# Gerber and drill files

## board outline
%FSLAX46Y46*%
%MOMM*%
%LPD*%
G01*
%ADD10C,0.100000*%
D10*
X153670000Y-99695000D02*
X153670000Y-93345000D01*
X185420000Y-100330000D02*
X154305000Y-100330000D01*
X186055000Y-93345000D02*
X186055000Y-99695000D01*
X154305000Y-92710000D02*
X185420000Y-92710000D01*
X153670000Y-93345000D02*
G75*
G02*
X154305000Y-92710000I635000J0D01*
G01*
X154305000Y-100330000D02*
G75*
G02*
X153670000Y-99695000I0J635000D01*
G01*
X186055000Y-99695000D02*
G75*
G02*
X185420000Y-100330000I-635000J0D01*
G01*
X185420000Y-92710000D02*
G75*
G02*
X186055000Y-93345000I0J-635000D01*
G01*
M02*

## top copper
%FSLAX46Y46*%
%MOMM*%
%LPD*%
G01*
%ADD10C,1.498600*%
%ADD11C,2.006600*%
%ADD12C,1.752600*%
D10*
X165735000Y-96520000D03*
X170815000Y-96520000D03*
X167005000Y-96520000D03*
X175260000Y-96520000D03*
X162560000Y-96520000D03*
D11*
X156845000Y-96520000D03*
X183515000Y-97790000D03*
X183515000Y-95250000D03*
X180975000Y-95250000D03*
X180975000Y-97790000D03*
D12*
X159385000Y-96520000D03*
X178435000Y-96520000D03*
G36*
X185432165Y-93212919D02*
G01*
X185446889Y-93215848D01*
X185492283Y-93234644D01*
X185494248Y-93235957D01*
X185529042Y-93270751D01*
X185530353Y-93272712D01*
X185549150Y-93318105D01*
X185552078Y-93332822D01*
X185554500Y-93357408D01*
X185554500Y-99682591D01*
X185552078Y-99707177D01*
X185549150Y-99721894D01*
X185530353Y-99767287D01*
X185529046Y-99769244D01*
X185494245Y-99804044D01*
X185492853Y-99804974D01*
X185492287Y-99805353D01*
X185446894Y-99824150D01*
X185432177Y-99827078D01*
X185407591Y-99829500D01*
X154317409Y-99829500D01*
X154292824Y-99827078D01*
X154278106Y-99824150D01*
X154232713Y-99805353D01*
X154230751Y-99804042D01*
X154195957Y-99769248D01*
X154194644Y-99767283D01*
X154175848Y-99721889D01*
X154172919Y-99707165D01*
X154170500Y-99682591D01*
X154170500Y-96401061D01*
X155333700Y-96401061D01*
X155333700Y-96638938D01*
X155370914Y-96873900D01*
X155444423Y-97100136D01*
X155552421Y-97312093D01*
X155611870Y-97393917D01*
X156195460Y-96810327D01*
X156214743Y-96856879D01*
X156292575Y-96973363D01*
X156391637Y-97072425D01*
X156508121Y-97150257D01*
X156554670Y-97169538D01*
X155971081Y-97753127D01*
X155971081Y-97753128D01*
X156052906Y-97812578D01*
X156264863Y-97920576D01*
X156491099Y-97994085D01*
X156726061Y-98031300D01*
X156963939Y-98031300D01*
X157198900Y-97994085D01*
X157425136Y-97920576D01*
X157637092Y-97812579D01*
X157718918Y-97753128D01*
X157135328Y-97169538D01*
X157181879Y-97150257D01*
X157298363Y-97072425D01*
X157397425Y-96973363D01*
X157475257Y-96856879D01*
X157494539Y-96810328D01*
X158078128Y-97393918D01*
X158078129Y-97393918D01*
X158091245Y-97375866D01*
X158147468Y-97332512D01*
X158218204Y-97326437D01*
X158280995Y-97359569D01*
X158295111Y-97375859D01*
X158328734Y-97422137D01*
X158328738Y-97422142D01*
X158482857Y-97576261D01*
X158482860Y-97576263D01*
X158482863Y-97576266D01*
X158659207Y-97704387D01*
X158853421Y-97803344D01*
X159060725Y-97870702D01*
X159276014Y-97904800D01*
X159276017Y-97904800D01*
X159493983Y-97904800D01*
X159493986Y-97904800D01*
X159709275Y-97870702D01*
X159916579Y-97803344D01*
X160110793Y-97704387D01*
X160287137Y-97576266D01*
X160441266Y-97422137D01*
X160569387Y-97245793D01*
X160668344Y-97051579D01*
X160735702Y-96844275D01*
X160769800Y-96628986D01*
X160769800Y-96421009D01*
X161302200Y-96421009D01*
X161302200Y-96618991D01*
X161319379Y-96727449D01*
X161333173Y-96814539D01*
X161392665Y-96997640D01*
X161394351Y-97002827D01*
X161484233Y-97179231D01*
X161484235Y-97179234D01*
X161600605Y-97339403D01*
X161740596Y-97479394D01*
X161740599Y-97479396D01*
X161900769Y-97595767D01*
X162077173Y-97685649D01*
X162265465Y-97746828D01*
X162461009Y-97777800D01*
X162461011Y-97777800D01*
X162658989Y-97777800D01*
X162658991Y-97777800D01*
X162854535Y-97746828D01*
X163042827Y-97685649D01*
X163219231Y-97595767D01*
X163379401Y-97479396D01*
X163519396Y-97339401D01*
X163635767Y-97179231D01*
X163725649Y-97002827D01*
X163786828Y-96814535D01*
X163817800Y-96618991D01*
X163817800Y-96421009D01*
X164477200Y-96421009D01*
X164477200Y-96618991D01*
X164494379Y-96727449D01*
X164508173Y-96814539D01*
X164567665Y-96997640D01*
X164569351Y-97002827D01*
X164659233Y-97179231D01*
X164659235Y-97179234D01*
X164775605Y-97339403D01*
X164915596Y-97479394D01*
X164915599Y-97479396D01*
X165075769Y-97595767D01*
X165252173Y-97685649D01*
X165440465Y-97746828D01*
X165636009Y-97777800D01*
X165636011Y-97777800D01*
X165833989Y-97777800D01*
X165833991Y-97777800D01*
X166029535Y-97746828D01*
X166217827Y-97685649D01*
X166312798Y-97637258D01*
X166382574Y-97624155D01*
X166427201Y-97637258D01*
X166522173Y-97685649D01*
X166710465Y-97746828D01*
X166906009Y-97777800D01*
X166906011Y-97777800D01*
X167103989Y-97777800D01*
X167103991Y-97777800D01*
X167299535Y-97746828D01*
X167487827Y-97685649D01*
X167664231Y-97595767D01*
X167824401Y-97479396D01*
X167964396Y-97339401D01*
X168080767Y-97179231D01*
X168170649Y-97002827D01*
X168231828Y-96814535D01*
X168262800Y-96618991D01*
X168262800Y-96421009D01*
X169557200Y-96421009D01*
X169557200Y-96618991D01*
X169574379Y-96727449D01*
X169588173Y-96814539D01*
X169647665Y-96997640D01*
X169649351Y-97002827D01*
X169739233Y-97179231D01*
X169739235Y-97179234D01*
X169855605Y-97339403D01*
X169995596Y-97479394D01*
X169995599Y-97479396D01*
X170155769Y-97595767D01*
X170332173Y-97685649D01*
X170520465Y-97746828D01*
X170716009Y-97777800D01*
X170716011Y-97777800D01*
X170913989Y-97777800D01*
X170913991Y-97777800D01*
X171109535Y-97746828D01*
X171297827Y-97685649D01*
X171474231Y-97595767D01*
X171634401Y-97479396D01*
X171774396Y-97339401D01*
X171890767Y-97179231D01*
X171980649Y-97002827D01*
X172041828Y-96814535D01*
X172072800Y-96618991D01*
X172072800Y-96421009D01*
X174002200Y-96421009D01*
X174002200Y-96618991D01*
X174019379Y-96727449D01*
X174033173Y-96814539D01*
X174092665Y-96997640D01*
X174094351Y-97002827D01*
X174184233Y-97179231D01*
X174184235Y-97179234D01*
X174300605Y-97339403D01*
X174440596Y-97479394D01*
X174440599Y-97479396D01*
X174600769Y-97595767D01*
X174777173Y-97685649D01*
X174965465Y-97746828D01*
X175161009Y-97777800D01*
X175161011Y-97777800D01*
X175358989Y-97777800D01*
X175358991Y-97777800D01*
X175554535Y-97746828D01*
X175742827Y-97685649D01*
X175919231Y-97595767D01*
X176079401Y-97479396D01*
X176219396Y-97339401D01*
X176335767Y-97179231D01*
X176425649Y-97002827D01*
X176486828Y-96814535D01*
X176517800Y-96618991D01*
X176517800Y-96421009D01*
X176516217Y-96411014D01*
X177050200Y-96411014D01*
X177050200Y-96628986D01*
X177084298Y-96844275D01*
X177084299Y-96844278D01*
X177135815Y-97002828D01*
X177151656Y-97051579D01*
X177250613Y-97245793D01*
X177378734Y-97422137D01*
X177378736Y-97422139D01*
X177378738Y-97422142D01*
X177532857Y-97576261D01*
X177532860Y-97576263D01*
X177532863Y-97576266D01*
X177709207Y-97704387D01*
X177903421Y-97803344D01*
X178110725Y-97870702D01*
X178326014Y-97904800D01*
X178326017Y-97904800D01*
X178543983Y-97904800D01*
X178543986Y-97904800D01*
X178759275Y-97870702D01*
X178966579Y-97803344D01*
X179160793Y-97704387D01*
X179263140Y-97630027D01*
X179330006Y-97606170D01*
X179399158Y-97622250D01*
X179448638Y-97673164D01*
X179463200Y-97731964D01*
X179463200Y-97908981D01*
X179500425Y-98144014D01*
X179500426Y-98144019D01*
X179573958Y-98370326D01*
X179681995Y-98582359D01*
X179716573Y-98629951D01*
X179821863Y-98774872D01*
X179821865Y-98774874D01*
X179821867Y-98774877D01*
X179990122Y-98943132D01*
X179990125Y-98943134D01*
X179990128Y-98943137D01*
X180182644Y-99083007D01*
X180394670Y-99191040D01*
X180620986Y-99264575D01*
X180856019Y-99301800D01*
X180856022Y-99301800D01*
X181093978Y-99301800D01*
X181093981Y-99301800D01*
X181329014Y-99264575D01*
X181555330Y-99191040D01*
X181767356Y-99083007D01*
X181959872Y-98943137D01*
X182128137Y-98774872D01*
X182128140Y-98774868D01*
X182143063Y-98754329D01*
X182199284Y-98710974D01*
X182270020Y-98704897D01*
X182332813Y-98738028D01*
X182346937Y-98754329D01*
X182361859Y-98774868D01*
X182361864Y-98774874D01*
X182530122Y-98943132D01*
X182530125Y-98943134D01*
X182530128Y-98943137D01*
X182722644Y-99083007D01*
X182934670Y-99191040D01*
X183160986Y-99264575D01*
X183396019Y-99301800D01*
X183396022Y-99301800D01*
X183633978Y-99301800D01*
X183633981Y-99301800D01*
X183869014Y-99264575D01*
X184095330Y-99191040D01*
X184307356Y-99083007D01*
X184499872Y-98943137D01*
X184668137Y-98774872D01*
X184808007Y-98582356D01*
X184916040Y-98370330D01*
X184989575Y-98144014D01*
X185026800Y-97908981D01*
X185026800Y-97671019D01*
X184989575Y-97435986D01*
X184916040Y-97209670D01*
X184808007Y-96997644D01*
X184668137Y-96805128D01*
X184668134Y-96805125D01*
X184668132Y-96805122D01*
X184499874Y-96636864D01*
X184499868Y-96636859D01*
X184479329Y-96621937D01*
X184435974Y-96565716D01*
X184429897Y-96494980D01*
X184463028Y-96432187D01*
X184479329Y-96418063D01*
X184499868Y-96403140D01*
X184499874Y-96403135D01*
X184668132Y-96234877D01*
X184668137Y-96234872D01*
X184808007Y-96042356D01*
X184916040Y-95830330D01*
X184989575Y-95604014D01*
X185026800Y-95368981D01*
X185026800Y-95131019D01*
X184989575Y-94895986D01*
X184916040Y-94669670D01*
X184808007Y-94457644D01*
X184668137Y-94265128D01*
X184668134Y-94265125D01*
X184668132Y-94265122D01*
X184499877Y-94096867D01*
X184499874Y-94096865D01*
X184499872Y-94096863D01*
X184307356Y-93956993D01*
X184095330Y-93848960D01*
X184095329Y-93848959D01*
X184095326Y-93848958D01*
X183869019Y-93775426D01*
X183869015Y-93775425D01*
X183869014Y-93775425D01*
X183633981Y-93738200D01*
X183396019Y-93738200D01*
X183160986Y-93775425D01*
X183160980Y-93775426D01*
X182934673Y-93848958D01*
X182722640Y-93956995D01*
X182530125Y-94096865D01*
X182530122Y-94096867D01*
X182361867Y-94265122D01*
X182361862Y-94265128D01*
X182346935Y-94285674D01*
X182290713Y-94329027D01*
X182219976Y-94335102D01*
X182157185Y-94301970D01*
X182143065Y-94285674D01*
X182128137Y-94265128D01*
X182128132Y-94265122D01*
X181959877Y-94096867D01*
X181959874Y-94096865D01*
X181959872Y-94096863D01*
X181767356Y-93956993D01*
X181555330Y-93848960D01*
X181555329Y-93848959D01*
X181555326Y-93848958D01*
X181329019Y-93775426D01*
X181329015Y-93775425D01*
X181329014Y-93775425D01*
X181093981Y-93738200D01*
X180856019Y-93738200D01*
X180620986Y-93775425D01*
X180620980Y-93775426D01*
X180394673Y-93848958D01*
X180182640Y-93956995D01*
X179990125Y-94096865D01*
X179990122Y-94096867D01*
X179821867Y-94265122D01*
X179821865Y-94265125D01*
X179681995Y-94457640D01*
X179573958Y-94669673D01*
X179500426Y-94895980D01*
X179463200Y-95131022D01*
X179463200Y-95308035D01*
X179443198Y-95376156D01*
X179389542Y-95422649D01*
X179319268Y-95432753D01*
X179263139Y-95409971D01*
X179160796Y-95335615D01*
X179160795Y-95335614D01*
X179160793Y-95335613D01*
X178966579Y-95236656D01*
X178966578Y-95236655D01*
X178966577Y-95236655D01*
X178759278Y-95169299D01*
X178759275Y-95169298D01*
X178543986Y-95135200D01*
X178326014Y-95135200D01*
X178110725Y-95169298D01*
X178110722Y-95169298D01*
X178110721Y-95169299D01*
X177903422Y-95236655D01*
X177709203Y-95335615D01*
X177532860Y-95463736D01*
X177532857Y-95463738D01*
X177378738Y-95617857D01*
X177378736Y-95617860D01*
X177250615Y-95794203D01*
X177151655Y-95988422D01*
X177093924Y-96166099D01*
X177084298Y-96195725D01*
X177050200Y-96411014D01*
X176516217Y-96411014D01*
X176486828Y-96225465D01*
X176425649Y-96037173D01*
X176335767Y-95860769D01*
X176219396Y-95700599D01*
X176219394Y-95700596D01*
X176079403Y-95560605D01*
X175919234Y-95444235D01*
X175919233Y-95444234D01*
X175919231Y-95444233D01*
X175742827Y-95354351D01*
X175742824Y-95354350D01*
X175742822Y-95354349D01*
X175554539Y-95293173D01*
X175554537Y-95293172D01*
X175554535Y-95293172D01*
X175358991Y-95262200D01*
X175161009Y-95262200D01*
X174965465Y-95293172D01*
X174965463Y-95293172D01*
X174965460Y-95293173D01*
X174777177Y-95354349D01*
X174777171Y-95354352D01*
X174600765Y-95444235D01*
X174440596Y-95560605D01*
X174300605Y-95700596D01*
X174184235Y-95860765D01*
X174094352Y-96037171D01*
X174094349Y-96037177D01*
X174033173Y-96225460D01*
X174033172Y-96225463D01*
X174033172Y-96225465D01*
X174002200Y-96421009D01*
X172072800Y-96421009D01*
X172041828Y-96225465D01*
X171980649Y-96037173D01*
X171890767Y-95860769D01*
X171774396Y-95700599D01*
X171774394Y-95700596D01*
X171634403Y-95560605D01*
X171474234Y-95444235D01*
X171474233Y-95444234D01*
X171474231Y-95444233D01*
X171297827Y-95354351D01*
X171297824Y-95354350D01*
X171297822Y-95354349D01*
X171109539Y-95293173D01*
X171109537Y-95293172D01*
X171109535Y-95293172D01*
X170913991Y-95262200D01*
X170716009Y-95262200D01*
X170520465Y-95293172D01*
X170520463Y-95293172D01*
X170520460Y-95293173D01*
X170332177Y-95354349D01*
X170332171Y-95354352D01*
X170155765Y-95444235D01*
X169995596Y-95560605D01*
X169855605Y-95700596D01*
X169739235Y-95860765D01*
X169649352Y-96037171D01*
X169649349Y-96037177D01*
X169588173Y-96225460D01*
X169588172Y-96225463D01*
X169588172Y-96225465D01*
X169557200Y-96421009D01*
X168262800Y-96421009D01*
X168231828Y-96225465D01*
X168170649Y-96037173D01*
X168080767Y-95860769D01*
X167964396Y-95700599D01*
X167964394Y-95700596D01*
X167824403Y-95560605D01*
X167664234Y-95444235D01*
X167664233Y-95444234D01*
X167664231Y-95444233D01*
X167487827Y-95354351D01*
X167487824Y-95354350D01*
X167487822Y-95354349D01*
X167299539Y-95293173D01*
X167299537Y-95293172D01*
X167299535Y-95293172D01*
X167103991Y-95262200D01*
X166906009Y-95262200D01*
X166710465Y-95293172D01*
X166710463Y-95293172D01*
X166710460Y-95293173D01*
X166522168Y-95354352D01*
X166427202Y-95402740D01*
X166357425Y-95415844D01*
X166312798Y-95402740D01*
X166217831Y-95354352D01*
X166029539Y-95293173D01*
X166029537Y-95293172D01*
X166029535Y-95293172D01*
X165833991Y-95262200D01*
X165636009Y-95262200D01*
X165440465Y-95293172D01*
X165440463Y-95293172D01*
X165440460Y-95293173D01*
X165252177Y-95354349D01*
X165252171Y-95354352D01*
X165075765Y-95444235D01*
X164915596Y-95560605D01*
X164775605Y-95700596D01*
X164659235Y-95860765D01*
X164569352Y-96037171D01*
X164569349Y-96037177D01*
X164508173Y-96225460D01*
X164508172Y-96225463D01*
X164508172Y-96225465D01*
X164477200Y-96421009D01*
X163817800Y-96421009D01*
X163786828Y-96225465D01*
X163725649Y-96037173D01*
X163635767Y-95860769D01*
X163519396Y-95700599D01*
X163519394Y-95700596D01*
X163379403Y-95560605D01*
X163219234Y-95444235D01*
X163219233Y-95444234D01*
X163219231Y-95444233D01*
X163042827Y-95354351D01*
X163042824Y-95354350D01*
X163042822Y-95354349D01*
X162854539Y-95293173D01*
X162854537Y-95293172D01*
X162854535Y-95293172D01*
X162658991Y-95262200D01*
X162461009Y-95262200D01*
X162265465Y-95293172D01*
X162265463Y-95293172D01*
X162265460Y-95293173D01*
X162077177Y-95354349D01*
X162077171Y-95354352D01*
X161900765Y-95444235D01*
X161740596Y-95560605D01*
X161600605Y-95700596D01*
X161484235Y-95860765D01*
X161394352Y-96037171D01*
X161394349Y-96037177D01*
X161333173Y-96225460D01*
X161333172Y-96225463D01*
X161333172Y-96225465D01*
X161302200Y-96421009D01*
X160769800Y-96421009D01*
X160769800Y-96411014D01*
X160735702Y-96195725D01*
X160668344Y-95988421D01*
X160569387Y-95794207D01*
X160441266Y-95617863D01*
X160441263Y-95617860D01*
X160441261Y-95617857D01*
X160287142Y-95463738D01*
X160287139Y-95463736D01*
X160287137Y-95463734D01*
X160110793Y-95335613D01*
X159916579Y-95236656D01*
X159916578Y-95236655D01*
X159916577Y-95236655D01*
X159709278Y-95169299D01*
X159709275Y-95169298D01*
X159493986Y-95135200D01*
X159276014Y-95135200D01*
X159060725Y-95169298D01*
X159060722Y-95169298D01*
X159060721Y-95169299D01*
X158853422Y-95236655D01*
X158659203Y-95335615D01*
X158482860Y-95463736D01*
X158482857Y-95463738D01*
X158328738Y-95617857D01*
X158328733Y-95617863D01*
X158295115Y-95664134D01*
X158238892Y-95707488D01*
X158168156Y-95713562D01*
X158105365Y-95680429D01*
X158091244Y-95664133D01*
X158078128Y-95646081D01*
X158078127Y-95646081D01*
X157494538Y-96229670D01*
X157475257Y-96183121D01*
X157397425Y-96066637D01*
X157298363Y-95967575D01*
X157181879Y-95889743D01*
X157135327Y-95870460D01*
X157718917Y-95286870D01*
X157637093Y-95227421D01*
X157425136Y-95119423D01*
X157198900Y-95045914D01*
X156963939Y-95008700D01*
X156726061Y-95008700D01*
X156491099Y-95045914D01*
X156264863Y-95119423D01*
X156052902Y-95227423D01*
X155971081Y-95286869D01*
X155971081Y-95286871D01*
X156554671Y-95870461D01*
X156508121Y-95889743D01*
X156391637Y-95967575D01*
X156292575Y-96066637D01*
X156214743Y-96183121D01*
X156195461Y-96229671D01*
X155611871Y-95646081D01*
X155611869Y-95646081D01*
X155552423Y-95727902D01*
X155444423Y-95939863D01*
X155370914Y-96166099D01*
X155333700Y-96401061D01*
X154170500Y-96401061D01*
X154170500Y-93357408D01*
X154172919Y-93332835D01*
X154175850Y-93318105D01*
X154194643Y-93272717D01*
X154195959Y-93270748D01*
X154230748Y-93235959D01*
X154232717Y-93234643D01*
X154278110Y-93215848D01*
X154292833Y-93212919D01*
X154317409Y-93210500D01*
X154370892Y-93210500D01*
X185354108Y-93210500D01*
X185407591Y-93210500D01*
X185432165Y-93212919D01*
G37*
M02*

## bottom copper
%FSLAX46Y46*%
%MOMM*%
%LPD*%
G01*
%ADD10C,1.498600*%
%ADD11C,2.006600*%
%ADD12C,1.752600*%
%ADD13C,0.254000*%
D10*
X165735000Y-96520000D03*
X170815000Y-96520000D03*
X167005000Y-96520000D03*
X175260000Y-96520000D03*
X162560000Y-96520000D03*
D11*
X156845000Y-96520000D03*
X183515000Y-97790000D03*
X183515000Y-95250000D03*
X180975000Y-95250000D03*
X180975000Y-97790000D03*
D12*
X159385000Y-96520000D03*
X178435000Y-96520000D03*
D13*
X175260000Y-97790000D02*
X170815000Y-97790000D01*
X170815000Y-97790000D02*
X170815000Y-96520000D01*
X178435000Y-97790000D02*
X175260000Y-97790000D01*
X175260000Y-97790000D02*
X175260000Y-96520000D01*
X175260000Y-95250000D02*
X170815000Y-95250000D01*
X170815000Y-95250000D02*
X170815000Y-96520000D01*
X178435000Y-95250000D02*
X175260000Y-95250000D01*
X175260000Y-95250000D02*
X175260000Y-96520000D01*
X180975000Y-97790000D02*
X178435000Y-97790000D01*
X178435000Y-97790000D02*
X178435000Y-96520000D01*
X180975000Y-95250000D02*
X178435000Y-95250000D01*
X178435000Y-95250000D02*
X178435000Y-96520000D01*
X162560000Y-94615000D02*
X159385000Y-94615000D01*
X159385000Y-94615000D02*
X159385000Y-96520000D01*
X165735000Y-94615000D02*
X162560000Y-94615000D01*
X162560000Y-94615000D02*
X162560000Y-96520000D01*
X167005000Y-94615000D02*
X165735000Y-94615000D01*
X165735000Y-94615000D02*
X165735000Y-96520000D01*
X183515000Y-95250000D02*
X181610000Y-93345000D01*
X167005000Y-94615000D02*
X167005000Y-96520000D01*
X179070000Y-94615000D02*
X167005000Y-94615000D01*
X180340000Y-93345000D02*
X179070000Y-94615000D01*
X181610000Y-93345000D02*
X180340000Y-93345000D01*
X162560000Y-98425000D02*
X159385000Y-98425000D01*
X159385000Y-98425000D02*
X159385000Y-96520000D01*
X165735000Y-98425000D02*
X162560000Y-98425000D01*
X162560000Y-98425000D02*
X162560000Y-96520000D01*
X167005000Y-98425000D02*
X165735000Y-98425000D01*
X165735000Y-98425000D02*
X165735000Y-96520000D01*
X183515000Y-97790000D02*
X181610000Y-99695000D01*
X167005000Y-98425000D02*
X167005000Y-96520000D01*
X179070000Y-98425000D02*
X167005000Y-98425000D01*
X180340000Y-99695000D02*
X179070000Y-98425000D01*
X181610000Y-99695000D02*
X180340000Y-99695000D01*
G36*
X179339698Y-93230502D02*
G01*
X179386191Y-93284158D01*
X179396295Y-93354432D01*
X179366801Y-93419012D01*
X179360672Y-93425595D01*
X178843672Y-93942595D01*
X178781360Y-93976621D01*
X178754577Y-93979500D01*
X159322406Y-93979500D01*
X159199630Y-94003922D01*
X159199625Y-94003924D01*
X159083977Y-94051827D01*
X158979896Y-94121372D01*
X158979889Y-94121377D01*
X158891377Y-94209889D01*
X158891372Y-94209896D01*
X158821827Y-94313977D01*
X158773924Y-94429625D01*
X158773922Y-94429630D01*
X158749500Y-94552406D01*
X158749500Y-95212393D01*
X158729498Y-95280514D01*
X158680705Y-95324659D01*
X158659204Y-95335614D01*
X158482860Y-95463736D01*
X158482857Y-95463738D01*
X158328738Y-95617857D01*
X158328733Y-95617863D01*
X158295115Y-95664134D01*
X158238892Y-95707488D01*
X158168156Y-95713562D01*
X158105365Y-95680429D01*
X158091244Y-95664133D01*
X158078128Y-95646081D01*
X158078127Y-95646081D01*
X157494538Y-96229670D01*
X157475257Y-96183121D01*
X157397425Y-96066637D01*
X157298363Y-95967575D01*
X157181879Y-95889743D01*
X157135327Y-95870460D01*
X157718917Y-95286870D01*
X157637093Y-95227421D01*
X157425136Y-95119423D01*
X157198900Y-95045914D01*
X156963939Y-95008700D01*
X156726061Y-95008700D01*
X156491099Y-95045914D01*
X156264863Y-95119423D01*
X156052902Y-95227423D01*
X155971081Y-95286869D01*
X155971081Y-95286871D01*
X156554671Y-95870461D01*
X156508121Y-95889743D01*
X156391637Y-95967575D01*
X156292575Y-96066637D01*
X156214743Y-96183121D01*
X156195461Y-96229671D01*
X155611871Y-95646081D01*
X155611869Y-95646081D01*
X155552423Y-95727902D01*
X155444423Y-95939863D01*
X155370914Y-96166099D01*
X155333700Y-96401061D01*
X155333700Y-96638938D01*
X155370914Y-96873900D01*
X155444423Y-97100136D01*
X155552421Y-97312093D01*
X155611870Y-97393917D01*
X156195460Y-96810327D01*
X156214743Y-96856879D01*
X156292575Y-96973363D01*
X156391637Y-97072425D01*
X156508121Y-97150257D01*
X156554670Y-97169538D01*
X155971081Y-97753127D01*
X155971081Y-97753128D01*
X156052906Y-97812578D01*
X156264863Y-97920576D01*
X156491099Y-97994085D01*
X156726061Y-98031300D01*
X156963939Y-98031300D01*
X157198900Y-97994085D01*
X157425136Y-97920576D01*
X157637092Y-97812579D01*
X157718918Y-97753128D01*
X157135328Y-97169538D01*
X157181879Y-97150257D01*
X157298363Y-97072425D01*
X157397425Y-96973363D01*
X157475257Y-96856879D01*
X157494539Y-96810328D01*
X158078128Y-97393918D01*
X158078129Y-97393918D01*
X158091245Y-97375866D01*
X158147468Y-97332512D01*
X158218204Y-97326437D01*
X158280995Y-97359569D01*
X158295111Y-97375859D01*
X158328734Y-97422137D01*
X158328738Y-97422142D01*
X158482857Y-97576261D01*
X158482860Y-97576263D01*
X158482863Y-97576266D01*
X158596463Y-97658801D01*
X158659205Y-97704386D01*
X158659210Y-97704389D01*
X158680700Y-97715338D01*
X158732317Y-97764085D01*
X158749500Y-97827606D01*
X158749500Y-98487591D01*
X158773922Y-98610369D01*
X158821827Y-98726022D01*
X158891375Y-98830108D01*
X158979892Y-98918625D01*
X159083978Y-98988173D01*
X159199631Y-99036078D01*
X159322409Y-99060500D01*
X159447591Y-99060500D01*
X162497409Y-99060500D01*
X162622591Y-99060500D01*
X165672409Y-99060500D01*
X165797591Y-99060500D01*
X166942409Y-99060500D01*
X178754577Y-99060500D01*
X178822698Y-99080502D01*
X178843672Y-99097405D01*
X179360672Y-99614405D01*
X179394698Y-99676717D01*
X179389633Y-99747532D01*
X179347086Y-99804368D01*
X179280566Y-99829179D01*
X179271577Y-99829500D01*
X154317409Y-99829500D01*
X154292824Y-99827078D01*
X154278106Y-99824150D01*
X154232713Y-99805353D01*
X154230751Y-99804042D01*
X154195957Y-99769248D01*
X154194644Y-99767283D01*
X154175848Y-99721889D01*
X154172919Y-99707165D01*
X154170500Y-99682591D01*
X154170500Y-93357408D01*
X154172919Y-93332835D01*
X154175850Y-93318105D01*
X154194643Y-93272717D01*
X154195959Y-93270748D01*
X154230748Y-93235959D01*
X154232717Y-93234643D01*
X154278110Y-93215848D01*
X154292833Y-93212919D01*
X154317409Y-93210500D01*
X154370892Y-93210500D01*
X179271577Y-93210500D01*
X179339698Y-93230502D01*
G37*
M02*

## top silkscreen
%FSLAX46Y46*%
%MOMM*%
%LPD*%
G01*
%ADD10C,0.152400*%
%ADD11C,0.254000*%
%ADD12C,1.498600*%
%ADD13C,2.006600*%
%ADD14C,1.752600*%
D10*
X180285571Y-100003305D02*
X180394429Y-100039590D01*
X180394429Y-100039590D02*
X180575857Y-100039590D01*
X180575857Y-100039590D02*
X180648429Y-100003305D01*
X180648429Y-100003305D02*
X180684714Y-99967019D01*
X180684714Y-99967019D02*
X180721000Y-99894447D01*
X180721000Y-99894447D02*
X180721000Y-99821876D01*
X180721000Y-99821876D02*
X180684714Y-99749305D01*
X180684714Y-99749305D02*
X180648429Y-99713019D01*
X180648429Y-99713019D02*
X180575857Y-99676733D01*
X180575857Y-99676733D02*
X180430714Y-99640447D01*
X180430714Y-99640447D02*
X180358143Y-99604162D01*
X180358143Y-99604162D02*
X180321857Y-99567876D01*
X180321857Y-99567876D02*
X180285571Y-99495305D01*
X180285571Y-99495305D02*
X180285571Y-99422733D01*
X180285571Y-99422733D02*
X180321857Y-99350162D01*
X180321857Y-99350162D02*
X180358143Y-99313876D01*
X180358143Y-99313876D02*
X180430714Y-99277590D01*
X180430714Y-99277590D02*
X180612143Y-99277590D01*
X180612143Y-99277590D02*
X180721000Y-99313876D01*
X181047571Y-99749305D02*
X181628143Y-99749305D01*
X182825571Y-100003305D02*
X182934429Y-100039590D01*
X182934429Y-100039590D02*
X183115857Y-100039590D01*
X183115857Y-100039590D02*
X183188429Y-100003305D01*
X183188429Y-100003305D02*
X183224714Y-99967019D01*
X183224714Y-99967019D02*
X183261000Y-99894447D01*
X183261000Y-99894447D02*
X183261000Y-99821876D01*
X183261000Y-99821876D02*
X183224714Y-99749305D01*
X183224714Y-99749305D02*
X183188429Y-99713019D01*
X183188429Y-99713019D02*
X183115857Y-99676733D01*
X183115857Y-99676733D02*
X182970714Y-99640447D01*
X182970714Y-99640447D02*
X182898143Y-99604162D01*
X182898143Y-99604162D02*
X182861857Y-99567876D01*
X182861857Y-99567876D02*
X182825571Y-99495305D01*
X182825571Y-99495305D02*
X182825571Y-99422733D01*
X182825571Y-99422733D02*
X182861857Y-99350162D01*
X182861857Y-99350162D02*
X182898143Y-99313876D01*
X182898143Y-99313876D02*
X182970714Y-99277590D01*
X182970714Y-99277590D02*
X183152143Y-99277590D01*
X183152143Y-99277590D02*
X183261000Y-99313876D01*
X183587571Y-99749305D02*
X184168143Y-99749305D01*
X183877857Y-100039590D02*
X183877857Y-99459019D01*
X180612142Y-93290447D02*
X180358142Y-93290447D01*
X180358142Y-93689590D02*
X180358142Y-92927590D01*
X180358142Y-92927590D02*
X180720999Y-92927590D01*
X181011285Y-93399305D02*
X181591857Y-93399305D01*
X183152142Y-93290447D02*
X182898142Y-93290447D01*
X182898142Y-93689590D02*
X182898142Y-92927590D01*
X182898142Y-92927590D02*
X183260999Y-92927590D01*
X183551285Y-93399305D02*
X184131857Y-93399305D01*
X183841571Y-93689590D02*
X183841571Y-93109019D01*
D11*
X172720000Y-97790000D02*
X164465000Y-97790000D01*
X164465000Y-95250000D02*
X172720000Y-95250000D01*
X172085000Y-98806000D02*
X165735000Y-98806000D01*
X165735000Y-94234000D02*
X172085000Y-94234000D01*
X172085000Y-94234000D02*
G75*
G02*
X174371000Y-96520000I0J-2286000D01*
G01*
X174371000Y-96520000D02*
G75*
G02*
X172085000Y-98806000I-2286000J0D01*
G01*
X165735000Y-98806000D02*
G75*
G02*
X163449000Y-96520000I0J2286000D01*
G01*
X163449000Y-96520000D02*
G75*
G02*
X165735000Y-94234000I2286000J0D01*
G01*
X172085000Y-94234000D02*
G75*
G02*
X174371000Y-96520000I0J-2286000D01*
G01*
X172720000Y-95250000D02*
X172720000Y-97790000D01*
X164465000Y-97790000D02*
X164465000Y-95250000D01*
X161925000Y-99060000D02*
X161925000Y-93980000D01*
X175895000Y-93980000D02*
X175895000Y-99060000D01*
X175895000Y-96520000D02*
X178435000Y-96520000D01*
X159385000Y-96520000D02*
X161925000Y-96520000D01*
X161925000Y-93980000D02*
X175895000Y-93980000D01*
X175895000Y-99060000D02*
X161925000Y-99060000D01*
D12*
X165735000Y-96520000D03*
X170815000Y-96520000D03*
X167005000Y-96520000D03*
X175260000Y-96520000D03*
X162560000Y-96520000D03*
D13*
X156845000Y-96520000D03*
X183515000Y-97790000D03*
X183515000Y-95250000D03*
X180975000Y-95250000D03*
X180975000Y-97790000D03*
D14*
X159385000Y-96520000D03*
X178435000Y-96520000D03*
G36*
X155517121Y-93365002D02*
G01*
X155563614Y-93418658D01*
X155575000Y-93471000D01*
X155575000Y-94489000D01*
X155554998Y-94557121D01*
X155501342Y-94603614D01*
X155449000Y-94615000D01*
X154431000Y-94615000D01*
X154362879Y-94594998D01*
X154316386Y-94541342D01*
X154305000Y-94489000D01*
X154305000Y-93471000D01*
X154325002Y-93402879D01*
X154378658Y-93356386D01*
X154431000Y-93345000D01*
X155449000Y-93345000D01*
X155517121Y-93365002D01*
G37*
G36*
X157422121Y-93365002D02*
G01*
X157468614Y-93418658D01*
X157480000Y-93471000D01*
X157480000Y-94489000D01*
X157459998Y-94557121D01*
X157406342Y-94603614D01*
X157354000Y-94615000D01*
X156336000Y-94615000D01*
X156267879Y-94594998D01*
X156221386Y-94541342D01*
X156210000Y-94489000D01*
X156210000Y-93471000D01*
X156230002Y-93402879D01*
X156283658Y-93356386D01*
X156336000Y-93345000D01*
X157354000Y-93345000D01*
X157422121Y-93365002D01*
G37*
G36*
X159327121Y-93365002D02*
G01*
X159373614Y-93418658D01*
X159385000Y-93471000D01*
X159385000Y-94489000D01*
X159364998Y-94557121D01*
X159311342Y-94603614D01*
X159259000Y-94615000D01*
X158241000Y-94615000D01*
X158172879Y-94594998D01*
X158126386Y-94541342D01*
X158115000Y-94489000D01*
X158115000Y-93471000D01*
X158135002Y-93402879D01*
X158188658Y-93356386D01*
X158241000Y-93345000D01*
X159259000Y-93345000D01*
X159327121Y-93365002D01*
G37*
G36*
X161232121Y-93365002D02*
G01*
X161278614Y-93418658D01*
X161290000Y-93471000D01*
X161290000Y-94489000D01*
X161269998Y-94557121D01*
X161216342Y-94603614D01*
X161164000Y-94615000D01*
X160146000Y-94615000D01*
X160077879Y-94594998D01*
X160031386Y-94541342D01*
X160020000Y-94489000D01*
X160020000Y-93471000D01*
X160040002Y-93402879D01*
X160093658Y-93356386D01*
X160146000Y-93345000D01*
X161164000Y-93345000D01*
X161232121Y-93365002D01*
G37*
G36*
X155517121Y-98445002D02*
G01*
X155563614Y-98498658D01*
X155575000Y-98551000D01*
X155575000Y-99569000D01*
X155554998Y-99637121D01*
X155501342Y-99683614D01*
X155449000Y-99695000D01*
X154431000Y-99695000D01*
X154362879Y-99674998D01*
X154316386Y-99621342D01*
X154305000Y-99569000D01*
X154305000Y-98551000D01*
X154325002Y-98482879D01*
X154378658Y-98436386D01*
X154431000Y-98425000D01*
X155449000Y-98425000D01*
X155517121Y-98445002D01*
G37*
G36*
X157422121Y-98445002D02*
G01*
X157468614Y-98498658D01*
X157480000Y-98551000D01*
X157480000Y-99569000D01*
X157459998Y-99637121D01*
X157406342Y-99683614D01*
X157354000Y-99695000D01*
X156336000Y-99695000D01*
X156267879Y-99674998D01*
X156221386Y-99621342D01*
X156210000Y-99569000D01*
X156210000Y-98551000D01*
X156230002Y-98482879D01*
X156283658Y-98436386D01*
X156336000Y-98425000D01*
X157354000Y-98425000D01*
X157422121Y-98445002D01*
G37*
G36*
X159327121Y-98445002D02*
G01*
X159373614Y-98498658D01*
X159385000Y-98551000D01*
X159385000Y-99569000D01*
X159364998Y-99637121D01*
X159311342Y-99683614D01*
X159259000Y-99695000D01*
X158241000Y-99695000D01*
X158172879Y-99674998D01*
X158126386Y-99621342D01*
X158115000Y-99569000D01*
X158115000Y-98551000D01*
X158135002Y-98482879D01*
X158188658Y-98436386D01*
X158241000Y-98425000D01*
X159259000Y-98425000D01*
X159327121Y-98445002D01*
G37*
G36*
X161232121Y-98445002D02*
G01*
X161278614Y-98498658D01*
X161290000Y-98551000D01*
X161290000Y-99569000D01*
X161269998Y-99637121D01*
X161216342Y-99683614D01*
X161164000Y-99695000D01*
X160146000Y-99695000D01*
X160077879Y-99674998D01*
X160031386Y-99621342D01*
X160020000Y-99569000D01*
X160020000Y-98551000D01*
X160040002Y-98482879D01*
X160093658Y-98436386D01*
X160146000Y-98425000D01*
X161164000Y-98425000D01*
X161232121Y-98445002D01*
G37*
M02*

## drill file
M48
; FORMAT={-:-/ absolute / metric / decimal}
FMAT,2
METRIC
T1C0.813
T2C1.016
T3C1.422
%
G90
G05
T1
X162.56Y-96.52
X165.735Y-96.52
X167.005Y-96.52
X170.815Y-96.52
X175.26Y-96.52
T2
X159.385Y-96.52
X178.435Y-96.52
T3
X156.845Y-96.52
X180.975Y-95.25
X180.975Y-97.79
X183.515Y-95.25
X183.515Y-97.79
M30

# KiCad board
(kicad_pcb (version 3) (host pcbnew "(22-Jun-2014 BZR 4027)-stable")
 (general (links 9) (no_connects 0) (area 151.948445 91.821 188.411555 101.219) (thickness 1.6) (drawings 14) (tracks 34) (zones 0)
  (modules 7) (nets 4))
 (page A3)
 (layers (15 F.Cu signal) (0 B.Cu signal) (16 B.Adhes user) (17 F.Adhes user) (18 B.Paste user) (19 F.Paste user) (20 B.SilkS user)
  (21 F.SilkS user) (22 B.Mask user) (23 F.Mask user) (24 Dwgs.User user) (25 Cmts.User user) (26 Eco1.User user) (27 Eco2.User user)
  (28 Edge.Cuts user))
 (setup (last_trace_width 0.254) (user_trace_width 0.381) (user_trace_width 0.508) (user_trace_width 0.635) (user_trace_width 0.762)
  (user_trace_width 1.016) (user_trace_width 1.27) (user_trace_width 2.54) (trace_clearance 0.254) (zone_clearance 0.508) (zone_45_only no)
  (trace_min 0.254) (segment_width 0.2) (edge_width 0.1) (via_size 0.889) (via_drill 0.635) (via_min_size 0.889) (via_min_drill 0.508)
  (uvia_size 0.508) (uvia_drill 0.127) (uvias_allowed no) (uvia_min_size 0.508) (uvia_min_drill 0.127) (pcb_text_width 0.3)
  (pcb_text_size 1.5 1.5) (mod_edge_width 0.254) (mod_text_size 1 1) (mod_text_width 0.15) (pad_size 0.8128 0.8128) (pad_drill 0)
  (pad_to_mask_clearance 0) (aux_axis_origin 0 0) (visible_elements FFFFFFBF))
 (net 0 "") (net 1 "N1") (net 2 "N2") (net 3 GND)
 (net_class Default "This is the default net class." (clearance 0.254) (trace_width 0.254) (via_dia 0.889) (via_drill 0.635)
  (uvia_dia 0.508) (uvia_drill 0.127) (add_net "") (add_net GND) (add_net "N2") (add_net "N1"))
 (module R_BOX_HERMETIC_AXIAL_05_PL (layer F.Cu) (at 168.91 96.52)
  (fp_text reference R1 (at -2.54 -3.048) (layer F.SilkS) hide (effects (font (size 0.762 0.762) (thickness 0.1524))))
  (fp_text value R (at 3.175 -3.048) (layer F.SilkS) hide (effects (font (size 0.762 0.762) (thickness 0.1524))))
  (fp_line (start 3.81 1.27) (end -4.445 1.27) (layer F.SilkS) (width 0.254))
  (fp_line (start -4.445 -1.27) (end 3.81 -1.27) (layer F.SilkS) (width 0.254))
  (fp_line (start 3.175 2.286) (end -3.175 2.286) (layer F.SilkS) (width 0.254))
  (fp_line (start -3.175 -2.286) (end 3.175 -2.286) (layer F.SilkS) (width 0.254))
  (fp_arc (start 3.175 0) (end 3.175 -2.286) (angle 90) (layer F.SilkS) (width 0.254))
  (fp_arc (start 3.175 0) (end 5.461 0) (angle 90) (layer F.SilkS) (width 0.254))
  (fp_arc (start -3.175 0) (end -3.175 2.286) (angle 90) (layer F.SilkS) (width 0.254))
  (fp_arc (start -3.175 0) (end -5.461 0) (angle 90) (layer F.SilkS) (width 0.254))
  (fp_arc (start 3.175 0) (end 3.175 -2.286) (angle 90) (layer F.SilkS) (width 0.254))
  (fp_line (start 3.81 -1.27) (end 3.81 1.27) (layer F.SilkS) (width 0.254))
  (fp_line (start -4.445 1.27) (end -4.445 -1.27) (layer F.SilkS) (width 0.254))
  (pad 1 thru_hole circle (at -3.175 0) (size 1.4986 1.4986) (drill 0.8128) (layers *.Cu *.Mask F.SilkS) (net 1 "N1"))
  (pad 2 thru_hole circle (at 1.905 0) (size 1.4986 1.4986) (drill 0.8128) (layers *.Cu *.Mask F.SilkS) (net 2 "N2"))
  (pad 1 thru_hole circle (at -1.905 0) (size 1.4986 1.4986) (drill 0.8128) (layers *.Cu *.Mask F.SilkS) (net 1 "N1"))
  (pad 2 thru_hole circle (at 6.35 0) (size 1.4986 1.4986) (drill 0.8128) (layers *.Cu *.Mask F.SilkS) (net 2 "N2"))
  (pad 1 thru_hole circle (at -6.35 0) (size 1.4986 1.4986) (drill 0.8128) (layers *.Cu *.Mask F.SilkS) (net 1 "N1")))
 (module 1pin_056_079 (layer F.Cu) (at 156.845 96.52)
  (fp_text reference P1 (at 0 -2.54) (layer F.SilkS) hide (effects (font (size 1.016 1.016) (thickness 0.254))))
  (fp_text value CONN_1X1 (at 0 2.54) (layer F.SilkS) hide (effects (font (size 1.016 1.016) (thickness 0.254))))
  (pad 1 thru_hole circle (at 0 0) (size 2.0066 2.0066) (drill 1.4224) (layers *.Cu *.Mask F.SilkS) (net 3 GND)))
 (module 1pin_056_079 (layer F.Cu) (at 183.515 97.79)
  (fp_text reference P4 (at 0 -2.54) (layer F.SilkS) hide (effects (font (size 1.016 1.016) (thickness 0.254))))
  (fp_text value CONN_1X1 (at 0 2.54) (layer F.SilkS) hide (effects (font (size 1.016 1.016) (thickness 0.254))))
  (pad 1 thru_hole circle (at 0 0) (size 2.0066 2.0066) (drill 1.4224) (layers *.Cu *.Mask F.SilkS) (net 1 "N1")))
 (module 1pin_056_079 (layer F.Cu) (at 183.515 95.25)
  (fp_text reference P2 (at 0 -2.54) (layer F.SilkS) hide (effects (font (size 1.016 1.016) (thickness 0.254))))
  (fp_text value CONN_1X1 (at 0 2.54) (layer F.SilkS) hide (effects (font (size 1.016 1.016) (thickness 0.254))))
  (pad 1 thru_hole circle (at 0 0) (size 2.0066 2.0066) (drill 1.4224) (layers *.Cu *.Mask F.SilkS) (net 1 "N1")))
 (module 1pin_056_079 (layer F.Cu) (at 180.975 95.25)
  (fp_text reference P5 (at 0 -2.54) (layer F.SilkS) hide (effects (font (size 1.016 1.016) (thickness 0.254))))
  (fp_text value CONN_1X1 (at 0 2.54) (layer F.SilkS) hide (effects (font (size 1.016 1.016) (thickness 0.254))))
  (pad 1 thru_hole circle (at 0 0) (size 2.0066 2.0066) (drill 1.4224) (layers *.Cu *.Mask F.SilkS) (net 2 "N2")))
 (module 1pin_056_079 (layer F.Cu) (at 180.975 97.79)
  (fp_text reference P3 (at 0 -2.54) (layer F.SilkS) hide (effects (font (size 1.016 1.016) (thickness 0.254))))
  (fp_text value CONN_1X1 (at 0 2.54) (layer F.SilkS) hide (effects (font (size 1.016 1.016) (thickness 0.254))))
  (pad 1 thru_hole circle (at 0 0) (size 2.0066 2.0066) (drill 1.4224) (layers *.Cu *.Mask F.SilkS) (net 2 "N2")))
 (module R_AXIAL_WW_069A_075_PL (layer F.Cu) (at 159.385 96.52) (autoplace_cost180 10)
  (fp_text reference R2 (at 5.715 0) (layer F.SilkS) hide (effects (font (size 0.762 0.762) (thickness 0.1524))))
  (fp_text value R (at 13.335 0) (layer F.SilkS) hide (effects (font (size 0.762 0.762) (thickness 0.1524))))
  (fp_line (start 2.54 2.54) (end 2.54 -2.54) (layer F.SilkS) (width 0.254))
  (fp_line (start 16.51 -2.54) (end 16.51 2.54) (layer F.SilkS) (width 0.254))
  (fp_line (start 16.51 0) (end 19.05 0) (layer F.SilkS) (width 0.254))
  (fp_line (start 0 0) (end 2.54 0) (layer F.SilkS) (width 0.254))
  (fp_line (start 2.54 -2.54) (end 16.51 -2.54) (layer F.SilkS) (width 0.254))
  (fp_line (start 16.51 2.54) (end 2.54 2.54) (layer F.SilkS) (width 0.254))
  (pad 1 thru_hole circle (at 0 0) (size 1.7526 1.7526) (drill 1.016) (layers *.Cu *.Mask F.SilkS) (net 1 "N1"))
  (pad 2 thru_hole circle (at 19.05 0) (size 1.7526 1.7526) (drill 1.016) (layers *.Cu *.Mask F.SilkS) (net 2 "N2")))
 (gr_line (start 153.67 99.695) (end 153.67 93.345) (angle 90) (layer Edge.Cuts) (width 0.1))
 (gr_line (start 185.42 100.33) (end 154.305 100.33) (angle 90) (layer Edge.Cuts) (width 0.1))
 (gr_line (start 186.055 93.345) (end 186.055 99.695) (angle 90) (layer Edge.Cuts) (width 0.1))
 (gr_line (start 154.305 92.71) (end 185.42 92.71) (angle 90) (layer Edge.Cuts) (width 0.1))
 (gr_arc (start 154.305 93.345) (end 153.67 93.345) (angle 90) (layer Edge.Cuts) (width 0.1))
 (gr_arc (start 154.305 99.695) (end 154.305 100.33) (angle 90) (layer Edge.Cuts) (width 0.1))
 (gr_arc (start 185.42 99.695) (end 186.055 99.695) (angle 90) (layer Edge.Cuts) (width 0.1))
 (gr_arc (start 185.42 93.345) (end 185.42 92.71) (angle 90) (layer Edge.Cuts) (width 0.1))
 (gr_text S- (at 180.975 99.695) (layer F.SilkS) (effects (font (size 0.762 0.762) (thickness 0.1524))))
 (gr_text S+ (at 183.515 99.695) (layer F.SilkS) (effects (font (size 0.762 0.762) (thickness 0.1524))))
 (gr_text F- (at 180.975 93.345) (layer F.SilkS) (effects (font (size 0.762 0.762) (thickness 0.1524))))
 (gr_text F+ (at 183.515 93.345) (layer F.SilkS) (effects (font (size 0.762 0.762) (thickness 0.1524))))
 (segment (start 175.26 97.79) (end 170.815 97.79) (width 0.254) (layer B.Cu) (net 2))
 (segment (start 170.815 97.79) (end 170.815 96.52) (width 0.254) (layer B.Cu) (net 2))
 (segment (start 178.435 97.79) (end 175.26 97.79) (width 0.254) (layer B.Cu) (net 2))
 (segment (start 175.26 97.79) (end 175.26 96.52) (width 0.254) (layer B.Cu) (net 2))
 (segment (start 175.26 95.25) (end 170.815 95.25) (width 0.254) (layer B.Cu) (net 2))
 (segment (start 170.815 95.25) (end 170.815 96.52) (width 0.254) (layer B.Cu) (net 2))
 (segment (start 178.435 95.25) (end 175.26 95.25) (width 0.254) (layer B.Cu) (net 2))
 (segment (start 175.26 95.25) (end 175.26 96.52) (width 0.254) (layer B.Cu) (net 2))
 (segment (start 180.975 97.79) (end 178.435 97.79) (width 0.254) (layer B.Cu) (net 2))
 (segment (start 178.435 97.79) (end 178.435 96.52) (width 0.254) (layer B.Cu) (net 2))
 (segment (start 180.975 95.25) (end 178.435 95.25) (width 0.254) (layer B.Cu) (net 2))
 (segment (start 178.435 95.25) (end 178.435 96.52) (width 0.254) (layer B.Cu) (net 2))
 (segment (start 162.56 94.615) (end 159.385 94.615) (width 0.254) (layer B.Cu) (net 1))
 (segment (start 159.385 94.615) (end 159.385 96.52) (width 0.254) (layer B.Cu) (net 1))
 (segment (start 165.735 94.615) (end 162.56 94.615) (width 0.254) (layer B.Cu) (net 1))
 (segment (start 162.56 94.615) (end 162.56 96.52) (width 0.254) (layer B.Cu) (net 1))
 (segment (start 167.005 94.615) (end 165.735 94.615) (width 0.254) (layer B.Cu) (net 1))
 (segment (start 165.735 94.615) (end 165.735 96.52) (width 0.254) (layer B.Cu) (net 1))
 (segment (start 183.515 95.25) (end 181.61 93.345) (width 0.254) (layer B.Cu) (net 1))
 (segment (start 167.005 94.615) (end 167.005 96.52) (width 0.254) (layer B.Cu) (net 1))
 (segment (start 179.07 94.615) (end 167.005 94.615) (width 0.254) (layer B.Cu) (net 1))
 (segment (start 180.34 93.345) (end 179.07 94.615) (width 0.254) (layer B.Cu) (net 1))
 (segment (start 181.61 93.345) (end 180.34 93.345) (width 0.254) (layer B.Cu) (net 1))
 (segment (start 162.56 98.425) (end 159.385 98.425) (width 0.254) (layer B.Cu) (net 1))
 (segment (start 159.385 98.425) (end 159.385 96.52) (width 0.254) (layer B.Cu) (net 1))
 (segment (start 165.735 98.425) (end 162.56 98.425) (width 0.254) (layer B.Cu) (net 1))
 (segment (start 162.56 98.425) (end 162.56 96.52) (width 0.254) (layer B.Cu) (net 1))
 (segment (start 167.005 98.425) (end 165.735 98.425) (width 0.254) (layer B.Cu) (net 1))
 (segment (start 165.735 98.425) (end 165.735 96.52) (width 0.254) (layer B.Cu) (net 1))
 (segment (start 183.515 97.79) (end 181.61 99.695) (width 0.254) (layer B.Cu) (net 1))
 (segment (start 167.005 98.425) (end 167.005 96.52) (width 0.254) (layer B.Cu) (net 1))
 (segment (start 179.07 98.425) (end 167.005 98.425) (width 0.254) (layer B.Cu) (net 1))
 (segment (start 180.34 99.695) (end 179.07 98.425) (width 0.254) (layer B.Cu) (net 1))
 (segment (start 181.61 99.695) (end 180.34 99.695) (width 0.254) (layer B.Cu) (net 1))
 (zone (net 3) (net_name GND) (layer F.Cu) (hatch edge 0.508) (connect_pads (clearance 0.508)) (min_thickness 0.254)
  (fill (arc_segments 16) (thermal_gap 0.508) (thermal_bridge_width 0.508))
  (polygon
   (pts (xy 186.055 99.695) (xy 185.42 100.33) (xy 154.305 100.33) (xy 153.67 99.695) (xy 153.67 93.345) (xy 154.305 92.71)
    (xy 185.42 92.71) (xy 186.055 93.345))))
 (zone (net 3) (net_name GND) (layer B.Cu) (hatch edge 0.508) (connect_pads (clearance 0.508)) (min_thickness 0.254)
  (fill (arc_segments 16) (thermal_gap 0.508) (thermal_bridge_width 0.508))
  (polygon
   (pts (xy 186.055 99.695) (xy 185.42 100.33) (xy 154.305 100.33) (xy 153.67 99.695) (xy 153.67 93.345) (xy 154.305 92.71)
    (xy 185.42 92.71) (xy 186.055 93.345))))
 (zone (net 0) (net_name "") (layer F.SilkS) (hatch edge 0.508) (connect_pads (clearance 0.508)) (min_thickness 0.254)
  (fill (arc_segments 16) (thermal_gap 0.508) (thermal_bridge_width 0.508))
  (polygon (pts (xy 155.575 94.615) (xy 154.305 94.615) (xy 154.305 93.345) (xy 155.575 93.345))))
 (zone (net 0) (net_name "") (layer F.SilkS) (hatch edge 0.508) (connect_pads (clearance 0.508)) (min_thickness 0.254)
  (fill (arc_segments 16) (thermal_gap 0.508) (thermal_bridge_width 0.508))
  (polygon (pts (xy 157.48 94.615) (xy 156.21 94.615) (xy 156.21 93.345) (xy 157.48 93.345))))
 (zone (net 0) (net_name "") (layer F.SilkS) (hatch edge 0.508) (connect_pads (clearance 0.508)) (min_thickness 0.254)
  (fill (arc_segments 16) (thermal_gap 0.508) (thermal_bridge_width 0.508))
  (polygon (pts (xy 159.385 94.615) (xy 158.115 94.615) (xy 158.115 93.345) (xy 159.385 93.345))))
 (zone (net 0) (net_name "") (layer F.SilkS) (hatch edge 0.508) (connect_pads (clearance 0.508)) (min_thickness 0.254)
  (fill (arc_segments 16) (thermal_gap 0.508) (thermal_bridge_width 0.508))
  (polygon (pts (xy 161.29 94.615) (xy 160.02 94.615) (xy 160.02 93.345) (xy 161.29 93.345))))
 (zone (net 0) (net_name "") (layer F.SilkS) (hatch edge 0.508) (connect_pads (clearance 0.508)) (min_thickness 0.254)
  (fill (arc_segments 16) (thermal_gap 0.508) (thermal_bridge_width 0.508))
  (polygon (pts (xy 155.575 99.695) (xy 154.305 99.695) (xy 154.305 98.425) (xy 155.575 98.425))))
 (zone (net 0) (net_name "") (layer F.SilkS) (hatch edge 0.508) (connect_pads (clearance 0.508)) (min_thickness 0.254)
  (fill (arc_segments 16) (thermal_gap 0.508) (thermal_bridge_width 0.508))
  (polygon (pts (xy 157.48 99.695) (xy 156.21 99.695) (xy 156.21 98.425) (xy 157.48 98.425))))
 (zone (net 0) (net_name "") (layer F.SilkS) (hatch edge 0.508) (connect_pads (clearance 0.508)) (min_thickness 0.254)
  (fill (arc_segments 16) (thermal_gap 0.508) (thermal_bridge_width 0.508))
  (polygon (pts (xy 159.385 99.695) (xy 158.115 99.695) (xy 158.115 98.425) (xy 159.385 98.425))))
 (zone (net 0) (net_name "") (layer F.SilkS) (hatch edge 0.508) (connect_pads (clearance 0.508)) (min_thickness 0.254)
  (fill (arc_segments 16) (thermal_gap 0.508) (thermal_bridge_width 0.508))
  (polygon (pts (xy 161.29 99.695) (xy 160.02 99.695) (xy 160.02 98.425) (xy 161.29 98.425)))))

